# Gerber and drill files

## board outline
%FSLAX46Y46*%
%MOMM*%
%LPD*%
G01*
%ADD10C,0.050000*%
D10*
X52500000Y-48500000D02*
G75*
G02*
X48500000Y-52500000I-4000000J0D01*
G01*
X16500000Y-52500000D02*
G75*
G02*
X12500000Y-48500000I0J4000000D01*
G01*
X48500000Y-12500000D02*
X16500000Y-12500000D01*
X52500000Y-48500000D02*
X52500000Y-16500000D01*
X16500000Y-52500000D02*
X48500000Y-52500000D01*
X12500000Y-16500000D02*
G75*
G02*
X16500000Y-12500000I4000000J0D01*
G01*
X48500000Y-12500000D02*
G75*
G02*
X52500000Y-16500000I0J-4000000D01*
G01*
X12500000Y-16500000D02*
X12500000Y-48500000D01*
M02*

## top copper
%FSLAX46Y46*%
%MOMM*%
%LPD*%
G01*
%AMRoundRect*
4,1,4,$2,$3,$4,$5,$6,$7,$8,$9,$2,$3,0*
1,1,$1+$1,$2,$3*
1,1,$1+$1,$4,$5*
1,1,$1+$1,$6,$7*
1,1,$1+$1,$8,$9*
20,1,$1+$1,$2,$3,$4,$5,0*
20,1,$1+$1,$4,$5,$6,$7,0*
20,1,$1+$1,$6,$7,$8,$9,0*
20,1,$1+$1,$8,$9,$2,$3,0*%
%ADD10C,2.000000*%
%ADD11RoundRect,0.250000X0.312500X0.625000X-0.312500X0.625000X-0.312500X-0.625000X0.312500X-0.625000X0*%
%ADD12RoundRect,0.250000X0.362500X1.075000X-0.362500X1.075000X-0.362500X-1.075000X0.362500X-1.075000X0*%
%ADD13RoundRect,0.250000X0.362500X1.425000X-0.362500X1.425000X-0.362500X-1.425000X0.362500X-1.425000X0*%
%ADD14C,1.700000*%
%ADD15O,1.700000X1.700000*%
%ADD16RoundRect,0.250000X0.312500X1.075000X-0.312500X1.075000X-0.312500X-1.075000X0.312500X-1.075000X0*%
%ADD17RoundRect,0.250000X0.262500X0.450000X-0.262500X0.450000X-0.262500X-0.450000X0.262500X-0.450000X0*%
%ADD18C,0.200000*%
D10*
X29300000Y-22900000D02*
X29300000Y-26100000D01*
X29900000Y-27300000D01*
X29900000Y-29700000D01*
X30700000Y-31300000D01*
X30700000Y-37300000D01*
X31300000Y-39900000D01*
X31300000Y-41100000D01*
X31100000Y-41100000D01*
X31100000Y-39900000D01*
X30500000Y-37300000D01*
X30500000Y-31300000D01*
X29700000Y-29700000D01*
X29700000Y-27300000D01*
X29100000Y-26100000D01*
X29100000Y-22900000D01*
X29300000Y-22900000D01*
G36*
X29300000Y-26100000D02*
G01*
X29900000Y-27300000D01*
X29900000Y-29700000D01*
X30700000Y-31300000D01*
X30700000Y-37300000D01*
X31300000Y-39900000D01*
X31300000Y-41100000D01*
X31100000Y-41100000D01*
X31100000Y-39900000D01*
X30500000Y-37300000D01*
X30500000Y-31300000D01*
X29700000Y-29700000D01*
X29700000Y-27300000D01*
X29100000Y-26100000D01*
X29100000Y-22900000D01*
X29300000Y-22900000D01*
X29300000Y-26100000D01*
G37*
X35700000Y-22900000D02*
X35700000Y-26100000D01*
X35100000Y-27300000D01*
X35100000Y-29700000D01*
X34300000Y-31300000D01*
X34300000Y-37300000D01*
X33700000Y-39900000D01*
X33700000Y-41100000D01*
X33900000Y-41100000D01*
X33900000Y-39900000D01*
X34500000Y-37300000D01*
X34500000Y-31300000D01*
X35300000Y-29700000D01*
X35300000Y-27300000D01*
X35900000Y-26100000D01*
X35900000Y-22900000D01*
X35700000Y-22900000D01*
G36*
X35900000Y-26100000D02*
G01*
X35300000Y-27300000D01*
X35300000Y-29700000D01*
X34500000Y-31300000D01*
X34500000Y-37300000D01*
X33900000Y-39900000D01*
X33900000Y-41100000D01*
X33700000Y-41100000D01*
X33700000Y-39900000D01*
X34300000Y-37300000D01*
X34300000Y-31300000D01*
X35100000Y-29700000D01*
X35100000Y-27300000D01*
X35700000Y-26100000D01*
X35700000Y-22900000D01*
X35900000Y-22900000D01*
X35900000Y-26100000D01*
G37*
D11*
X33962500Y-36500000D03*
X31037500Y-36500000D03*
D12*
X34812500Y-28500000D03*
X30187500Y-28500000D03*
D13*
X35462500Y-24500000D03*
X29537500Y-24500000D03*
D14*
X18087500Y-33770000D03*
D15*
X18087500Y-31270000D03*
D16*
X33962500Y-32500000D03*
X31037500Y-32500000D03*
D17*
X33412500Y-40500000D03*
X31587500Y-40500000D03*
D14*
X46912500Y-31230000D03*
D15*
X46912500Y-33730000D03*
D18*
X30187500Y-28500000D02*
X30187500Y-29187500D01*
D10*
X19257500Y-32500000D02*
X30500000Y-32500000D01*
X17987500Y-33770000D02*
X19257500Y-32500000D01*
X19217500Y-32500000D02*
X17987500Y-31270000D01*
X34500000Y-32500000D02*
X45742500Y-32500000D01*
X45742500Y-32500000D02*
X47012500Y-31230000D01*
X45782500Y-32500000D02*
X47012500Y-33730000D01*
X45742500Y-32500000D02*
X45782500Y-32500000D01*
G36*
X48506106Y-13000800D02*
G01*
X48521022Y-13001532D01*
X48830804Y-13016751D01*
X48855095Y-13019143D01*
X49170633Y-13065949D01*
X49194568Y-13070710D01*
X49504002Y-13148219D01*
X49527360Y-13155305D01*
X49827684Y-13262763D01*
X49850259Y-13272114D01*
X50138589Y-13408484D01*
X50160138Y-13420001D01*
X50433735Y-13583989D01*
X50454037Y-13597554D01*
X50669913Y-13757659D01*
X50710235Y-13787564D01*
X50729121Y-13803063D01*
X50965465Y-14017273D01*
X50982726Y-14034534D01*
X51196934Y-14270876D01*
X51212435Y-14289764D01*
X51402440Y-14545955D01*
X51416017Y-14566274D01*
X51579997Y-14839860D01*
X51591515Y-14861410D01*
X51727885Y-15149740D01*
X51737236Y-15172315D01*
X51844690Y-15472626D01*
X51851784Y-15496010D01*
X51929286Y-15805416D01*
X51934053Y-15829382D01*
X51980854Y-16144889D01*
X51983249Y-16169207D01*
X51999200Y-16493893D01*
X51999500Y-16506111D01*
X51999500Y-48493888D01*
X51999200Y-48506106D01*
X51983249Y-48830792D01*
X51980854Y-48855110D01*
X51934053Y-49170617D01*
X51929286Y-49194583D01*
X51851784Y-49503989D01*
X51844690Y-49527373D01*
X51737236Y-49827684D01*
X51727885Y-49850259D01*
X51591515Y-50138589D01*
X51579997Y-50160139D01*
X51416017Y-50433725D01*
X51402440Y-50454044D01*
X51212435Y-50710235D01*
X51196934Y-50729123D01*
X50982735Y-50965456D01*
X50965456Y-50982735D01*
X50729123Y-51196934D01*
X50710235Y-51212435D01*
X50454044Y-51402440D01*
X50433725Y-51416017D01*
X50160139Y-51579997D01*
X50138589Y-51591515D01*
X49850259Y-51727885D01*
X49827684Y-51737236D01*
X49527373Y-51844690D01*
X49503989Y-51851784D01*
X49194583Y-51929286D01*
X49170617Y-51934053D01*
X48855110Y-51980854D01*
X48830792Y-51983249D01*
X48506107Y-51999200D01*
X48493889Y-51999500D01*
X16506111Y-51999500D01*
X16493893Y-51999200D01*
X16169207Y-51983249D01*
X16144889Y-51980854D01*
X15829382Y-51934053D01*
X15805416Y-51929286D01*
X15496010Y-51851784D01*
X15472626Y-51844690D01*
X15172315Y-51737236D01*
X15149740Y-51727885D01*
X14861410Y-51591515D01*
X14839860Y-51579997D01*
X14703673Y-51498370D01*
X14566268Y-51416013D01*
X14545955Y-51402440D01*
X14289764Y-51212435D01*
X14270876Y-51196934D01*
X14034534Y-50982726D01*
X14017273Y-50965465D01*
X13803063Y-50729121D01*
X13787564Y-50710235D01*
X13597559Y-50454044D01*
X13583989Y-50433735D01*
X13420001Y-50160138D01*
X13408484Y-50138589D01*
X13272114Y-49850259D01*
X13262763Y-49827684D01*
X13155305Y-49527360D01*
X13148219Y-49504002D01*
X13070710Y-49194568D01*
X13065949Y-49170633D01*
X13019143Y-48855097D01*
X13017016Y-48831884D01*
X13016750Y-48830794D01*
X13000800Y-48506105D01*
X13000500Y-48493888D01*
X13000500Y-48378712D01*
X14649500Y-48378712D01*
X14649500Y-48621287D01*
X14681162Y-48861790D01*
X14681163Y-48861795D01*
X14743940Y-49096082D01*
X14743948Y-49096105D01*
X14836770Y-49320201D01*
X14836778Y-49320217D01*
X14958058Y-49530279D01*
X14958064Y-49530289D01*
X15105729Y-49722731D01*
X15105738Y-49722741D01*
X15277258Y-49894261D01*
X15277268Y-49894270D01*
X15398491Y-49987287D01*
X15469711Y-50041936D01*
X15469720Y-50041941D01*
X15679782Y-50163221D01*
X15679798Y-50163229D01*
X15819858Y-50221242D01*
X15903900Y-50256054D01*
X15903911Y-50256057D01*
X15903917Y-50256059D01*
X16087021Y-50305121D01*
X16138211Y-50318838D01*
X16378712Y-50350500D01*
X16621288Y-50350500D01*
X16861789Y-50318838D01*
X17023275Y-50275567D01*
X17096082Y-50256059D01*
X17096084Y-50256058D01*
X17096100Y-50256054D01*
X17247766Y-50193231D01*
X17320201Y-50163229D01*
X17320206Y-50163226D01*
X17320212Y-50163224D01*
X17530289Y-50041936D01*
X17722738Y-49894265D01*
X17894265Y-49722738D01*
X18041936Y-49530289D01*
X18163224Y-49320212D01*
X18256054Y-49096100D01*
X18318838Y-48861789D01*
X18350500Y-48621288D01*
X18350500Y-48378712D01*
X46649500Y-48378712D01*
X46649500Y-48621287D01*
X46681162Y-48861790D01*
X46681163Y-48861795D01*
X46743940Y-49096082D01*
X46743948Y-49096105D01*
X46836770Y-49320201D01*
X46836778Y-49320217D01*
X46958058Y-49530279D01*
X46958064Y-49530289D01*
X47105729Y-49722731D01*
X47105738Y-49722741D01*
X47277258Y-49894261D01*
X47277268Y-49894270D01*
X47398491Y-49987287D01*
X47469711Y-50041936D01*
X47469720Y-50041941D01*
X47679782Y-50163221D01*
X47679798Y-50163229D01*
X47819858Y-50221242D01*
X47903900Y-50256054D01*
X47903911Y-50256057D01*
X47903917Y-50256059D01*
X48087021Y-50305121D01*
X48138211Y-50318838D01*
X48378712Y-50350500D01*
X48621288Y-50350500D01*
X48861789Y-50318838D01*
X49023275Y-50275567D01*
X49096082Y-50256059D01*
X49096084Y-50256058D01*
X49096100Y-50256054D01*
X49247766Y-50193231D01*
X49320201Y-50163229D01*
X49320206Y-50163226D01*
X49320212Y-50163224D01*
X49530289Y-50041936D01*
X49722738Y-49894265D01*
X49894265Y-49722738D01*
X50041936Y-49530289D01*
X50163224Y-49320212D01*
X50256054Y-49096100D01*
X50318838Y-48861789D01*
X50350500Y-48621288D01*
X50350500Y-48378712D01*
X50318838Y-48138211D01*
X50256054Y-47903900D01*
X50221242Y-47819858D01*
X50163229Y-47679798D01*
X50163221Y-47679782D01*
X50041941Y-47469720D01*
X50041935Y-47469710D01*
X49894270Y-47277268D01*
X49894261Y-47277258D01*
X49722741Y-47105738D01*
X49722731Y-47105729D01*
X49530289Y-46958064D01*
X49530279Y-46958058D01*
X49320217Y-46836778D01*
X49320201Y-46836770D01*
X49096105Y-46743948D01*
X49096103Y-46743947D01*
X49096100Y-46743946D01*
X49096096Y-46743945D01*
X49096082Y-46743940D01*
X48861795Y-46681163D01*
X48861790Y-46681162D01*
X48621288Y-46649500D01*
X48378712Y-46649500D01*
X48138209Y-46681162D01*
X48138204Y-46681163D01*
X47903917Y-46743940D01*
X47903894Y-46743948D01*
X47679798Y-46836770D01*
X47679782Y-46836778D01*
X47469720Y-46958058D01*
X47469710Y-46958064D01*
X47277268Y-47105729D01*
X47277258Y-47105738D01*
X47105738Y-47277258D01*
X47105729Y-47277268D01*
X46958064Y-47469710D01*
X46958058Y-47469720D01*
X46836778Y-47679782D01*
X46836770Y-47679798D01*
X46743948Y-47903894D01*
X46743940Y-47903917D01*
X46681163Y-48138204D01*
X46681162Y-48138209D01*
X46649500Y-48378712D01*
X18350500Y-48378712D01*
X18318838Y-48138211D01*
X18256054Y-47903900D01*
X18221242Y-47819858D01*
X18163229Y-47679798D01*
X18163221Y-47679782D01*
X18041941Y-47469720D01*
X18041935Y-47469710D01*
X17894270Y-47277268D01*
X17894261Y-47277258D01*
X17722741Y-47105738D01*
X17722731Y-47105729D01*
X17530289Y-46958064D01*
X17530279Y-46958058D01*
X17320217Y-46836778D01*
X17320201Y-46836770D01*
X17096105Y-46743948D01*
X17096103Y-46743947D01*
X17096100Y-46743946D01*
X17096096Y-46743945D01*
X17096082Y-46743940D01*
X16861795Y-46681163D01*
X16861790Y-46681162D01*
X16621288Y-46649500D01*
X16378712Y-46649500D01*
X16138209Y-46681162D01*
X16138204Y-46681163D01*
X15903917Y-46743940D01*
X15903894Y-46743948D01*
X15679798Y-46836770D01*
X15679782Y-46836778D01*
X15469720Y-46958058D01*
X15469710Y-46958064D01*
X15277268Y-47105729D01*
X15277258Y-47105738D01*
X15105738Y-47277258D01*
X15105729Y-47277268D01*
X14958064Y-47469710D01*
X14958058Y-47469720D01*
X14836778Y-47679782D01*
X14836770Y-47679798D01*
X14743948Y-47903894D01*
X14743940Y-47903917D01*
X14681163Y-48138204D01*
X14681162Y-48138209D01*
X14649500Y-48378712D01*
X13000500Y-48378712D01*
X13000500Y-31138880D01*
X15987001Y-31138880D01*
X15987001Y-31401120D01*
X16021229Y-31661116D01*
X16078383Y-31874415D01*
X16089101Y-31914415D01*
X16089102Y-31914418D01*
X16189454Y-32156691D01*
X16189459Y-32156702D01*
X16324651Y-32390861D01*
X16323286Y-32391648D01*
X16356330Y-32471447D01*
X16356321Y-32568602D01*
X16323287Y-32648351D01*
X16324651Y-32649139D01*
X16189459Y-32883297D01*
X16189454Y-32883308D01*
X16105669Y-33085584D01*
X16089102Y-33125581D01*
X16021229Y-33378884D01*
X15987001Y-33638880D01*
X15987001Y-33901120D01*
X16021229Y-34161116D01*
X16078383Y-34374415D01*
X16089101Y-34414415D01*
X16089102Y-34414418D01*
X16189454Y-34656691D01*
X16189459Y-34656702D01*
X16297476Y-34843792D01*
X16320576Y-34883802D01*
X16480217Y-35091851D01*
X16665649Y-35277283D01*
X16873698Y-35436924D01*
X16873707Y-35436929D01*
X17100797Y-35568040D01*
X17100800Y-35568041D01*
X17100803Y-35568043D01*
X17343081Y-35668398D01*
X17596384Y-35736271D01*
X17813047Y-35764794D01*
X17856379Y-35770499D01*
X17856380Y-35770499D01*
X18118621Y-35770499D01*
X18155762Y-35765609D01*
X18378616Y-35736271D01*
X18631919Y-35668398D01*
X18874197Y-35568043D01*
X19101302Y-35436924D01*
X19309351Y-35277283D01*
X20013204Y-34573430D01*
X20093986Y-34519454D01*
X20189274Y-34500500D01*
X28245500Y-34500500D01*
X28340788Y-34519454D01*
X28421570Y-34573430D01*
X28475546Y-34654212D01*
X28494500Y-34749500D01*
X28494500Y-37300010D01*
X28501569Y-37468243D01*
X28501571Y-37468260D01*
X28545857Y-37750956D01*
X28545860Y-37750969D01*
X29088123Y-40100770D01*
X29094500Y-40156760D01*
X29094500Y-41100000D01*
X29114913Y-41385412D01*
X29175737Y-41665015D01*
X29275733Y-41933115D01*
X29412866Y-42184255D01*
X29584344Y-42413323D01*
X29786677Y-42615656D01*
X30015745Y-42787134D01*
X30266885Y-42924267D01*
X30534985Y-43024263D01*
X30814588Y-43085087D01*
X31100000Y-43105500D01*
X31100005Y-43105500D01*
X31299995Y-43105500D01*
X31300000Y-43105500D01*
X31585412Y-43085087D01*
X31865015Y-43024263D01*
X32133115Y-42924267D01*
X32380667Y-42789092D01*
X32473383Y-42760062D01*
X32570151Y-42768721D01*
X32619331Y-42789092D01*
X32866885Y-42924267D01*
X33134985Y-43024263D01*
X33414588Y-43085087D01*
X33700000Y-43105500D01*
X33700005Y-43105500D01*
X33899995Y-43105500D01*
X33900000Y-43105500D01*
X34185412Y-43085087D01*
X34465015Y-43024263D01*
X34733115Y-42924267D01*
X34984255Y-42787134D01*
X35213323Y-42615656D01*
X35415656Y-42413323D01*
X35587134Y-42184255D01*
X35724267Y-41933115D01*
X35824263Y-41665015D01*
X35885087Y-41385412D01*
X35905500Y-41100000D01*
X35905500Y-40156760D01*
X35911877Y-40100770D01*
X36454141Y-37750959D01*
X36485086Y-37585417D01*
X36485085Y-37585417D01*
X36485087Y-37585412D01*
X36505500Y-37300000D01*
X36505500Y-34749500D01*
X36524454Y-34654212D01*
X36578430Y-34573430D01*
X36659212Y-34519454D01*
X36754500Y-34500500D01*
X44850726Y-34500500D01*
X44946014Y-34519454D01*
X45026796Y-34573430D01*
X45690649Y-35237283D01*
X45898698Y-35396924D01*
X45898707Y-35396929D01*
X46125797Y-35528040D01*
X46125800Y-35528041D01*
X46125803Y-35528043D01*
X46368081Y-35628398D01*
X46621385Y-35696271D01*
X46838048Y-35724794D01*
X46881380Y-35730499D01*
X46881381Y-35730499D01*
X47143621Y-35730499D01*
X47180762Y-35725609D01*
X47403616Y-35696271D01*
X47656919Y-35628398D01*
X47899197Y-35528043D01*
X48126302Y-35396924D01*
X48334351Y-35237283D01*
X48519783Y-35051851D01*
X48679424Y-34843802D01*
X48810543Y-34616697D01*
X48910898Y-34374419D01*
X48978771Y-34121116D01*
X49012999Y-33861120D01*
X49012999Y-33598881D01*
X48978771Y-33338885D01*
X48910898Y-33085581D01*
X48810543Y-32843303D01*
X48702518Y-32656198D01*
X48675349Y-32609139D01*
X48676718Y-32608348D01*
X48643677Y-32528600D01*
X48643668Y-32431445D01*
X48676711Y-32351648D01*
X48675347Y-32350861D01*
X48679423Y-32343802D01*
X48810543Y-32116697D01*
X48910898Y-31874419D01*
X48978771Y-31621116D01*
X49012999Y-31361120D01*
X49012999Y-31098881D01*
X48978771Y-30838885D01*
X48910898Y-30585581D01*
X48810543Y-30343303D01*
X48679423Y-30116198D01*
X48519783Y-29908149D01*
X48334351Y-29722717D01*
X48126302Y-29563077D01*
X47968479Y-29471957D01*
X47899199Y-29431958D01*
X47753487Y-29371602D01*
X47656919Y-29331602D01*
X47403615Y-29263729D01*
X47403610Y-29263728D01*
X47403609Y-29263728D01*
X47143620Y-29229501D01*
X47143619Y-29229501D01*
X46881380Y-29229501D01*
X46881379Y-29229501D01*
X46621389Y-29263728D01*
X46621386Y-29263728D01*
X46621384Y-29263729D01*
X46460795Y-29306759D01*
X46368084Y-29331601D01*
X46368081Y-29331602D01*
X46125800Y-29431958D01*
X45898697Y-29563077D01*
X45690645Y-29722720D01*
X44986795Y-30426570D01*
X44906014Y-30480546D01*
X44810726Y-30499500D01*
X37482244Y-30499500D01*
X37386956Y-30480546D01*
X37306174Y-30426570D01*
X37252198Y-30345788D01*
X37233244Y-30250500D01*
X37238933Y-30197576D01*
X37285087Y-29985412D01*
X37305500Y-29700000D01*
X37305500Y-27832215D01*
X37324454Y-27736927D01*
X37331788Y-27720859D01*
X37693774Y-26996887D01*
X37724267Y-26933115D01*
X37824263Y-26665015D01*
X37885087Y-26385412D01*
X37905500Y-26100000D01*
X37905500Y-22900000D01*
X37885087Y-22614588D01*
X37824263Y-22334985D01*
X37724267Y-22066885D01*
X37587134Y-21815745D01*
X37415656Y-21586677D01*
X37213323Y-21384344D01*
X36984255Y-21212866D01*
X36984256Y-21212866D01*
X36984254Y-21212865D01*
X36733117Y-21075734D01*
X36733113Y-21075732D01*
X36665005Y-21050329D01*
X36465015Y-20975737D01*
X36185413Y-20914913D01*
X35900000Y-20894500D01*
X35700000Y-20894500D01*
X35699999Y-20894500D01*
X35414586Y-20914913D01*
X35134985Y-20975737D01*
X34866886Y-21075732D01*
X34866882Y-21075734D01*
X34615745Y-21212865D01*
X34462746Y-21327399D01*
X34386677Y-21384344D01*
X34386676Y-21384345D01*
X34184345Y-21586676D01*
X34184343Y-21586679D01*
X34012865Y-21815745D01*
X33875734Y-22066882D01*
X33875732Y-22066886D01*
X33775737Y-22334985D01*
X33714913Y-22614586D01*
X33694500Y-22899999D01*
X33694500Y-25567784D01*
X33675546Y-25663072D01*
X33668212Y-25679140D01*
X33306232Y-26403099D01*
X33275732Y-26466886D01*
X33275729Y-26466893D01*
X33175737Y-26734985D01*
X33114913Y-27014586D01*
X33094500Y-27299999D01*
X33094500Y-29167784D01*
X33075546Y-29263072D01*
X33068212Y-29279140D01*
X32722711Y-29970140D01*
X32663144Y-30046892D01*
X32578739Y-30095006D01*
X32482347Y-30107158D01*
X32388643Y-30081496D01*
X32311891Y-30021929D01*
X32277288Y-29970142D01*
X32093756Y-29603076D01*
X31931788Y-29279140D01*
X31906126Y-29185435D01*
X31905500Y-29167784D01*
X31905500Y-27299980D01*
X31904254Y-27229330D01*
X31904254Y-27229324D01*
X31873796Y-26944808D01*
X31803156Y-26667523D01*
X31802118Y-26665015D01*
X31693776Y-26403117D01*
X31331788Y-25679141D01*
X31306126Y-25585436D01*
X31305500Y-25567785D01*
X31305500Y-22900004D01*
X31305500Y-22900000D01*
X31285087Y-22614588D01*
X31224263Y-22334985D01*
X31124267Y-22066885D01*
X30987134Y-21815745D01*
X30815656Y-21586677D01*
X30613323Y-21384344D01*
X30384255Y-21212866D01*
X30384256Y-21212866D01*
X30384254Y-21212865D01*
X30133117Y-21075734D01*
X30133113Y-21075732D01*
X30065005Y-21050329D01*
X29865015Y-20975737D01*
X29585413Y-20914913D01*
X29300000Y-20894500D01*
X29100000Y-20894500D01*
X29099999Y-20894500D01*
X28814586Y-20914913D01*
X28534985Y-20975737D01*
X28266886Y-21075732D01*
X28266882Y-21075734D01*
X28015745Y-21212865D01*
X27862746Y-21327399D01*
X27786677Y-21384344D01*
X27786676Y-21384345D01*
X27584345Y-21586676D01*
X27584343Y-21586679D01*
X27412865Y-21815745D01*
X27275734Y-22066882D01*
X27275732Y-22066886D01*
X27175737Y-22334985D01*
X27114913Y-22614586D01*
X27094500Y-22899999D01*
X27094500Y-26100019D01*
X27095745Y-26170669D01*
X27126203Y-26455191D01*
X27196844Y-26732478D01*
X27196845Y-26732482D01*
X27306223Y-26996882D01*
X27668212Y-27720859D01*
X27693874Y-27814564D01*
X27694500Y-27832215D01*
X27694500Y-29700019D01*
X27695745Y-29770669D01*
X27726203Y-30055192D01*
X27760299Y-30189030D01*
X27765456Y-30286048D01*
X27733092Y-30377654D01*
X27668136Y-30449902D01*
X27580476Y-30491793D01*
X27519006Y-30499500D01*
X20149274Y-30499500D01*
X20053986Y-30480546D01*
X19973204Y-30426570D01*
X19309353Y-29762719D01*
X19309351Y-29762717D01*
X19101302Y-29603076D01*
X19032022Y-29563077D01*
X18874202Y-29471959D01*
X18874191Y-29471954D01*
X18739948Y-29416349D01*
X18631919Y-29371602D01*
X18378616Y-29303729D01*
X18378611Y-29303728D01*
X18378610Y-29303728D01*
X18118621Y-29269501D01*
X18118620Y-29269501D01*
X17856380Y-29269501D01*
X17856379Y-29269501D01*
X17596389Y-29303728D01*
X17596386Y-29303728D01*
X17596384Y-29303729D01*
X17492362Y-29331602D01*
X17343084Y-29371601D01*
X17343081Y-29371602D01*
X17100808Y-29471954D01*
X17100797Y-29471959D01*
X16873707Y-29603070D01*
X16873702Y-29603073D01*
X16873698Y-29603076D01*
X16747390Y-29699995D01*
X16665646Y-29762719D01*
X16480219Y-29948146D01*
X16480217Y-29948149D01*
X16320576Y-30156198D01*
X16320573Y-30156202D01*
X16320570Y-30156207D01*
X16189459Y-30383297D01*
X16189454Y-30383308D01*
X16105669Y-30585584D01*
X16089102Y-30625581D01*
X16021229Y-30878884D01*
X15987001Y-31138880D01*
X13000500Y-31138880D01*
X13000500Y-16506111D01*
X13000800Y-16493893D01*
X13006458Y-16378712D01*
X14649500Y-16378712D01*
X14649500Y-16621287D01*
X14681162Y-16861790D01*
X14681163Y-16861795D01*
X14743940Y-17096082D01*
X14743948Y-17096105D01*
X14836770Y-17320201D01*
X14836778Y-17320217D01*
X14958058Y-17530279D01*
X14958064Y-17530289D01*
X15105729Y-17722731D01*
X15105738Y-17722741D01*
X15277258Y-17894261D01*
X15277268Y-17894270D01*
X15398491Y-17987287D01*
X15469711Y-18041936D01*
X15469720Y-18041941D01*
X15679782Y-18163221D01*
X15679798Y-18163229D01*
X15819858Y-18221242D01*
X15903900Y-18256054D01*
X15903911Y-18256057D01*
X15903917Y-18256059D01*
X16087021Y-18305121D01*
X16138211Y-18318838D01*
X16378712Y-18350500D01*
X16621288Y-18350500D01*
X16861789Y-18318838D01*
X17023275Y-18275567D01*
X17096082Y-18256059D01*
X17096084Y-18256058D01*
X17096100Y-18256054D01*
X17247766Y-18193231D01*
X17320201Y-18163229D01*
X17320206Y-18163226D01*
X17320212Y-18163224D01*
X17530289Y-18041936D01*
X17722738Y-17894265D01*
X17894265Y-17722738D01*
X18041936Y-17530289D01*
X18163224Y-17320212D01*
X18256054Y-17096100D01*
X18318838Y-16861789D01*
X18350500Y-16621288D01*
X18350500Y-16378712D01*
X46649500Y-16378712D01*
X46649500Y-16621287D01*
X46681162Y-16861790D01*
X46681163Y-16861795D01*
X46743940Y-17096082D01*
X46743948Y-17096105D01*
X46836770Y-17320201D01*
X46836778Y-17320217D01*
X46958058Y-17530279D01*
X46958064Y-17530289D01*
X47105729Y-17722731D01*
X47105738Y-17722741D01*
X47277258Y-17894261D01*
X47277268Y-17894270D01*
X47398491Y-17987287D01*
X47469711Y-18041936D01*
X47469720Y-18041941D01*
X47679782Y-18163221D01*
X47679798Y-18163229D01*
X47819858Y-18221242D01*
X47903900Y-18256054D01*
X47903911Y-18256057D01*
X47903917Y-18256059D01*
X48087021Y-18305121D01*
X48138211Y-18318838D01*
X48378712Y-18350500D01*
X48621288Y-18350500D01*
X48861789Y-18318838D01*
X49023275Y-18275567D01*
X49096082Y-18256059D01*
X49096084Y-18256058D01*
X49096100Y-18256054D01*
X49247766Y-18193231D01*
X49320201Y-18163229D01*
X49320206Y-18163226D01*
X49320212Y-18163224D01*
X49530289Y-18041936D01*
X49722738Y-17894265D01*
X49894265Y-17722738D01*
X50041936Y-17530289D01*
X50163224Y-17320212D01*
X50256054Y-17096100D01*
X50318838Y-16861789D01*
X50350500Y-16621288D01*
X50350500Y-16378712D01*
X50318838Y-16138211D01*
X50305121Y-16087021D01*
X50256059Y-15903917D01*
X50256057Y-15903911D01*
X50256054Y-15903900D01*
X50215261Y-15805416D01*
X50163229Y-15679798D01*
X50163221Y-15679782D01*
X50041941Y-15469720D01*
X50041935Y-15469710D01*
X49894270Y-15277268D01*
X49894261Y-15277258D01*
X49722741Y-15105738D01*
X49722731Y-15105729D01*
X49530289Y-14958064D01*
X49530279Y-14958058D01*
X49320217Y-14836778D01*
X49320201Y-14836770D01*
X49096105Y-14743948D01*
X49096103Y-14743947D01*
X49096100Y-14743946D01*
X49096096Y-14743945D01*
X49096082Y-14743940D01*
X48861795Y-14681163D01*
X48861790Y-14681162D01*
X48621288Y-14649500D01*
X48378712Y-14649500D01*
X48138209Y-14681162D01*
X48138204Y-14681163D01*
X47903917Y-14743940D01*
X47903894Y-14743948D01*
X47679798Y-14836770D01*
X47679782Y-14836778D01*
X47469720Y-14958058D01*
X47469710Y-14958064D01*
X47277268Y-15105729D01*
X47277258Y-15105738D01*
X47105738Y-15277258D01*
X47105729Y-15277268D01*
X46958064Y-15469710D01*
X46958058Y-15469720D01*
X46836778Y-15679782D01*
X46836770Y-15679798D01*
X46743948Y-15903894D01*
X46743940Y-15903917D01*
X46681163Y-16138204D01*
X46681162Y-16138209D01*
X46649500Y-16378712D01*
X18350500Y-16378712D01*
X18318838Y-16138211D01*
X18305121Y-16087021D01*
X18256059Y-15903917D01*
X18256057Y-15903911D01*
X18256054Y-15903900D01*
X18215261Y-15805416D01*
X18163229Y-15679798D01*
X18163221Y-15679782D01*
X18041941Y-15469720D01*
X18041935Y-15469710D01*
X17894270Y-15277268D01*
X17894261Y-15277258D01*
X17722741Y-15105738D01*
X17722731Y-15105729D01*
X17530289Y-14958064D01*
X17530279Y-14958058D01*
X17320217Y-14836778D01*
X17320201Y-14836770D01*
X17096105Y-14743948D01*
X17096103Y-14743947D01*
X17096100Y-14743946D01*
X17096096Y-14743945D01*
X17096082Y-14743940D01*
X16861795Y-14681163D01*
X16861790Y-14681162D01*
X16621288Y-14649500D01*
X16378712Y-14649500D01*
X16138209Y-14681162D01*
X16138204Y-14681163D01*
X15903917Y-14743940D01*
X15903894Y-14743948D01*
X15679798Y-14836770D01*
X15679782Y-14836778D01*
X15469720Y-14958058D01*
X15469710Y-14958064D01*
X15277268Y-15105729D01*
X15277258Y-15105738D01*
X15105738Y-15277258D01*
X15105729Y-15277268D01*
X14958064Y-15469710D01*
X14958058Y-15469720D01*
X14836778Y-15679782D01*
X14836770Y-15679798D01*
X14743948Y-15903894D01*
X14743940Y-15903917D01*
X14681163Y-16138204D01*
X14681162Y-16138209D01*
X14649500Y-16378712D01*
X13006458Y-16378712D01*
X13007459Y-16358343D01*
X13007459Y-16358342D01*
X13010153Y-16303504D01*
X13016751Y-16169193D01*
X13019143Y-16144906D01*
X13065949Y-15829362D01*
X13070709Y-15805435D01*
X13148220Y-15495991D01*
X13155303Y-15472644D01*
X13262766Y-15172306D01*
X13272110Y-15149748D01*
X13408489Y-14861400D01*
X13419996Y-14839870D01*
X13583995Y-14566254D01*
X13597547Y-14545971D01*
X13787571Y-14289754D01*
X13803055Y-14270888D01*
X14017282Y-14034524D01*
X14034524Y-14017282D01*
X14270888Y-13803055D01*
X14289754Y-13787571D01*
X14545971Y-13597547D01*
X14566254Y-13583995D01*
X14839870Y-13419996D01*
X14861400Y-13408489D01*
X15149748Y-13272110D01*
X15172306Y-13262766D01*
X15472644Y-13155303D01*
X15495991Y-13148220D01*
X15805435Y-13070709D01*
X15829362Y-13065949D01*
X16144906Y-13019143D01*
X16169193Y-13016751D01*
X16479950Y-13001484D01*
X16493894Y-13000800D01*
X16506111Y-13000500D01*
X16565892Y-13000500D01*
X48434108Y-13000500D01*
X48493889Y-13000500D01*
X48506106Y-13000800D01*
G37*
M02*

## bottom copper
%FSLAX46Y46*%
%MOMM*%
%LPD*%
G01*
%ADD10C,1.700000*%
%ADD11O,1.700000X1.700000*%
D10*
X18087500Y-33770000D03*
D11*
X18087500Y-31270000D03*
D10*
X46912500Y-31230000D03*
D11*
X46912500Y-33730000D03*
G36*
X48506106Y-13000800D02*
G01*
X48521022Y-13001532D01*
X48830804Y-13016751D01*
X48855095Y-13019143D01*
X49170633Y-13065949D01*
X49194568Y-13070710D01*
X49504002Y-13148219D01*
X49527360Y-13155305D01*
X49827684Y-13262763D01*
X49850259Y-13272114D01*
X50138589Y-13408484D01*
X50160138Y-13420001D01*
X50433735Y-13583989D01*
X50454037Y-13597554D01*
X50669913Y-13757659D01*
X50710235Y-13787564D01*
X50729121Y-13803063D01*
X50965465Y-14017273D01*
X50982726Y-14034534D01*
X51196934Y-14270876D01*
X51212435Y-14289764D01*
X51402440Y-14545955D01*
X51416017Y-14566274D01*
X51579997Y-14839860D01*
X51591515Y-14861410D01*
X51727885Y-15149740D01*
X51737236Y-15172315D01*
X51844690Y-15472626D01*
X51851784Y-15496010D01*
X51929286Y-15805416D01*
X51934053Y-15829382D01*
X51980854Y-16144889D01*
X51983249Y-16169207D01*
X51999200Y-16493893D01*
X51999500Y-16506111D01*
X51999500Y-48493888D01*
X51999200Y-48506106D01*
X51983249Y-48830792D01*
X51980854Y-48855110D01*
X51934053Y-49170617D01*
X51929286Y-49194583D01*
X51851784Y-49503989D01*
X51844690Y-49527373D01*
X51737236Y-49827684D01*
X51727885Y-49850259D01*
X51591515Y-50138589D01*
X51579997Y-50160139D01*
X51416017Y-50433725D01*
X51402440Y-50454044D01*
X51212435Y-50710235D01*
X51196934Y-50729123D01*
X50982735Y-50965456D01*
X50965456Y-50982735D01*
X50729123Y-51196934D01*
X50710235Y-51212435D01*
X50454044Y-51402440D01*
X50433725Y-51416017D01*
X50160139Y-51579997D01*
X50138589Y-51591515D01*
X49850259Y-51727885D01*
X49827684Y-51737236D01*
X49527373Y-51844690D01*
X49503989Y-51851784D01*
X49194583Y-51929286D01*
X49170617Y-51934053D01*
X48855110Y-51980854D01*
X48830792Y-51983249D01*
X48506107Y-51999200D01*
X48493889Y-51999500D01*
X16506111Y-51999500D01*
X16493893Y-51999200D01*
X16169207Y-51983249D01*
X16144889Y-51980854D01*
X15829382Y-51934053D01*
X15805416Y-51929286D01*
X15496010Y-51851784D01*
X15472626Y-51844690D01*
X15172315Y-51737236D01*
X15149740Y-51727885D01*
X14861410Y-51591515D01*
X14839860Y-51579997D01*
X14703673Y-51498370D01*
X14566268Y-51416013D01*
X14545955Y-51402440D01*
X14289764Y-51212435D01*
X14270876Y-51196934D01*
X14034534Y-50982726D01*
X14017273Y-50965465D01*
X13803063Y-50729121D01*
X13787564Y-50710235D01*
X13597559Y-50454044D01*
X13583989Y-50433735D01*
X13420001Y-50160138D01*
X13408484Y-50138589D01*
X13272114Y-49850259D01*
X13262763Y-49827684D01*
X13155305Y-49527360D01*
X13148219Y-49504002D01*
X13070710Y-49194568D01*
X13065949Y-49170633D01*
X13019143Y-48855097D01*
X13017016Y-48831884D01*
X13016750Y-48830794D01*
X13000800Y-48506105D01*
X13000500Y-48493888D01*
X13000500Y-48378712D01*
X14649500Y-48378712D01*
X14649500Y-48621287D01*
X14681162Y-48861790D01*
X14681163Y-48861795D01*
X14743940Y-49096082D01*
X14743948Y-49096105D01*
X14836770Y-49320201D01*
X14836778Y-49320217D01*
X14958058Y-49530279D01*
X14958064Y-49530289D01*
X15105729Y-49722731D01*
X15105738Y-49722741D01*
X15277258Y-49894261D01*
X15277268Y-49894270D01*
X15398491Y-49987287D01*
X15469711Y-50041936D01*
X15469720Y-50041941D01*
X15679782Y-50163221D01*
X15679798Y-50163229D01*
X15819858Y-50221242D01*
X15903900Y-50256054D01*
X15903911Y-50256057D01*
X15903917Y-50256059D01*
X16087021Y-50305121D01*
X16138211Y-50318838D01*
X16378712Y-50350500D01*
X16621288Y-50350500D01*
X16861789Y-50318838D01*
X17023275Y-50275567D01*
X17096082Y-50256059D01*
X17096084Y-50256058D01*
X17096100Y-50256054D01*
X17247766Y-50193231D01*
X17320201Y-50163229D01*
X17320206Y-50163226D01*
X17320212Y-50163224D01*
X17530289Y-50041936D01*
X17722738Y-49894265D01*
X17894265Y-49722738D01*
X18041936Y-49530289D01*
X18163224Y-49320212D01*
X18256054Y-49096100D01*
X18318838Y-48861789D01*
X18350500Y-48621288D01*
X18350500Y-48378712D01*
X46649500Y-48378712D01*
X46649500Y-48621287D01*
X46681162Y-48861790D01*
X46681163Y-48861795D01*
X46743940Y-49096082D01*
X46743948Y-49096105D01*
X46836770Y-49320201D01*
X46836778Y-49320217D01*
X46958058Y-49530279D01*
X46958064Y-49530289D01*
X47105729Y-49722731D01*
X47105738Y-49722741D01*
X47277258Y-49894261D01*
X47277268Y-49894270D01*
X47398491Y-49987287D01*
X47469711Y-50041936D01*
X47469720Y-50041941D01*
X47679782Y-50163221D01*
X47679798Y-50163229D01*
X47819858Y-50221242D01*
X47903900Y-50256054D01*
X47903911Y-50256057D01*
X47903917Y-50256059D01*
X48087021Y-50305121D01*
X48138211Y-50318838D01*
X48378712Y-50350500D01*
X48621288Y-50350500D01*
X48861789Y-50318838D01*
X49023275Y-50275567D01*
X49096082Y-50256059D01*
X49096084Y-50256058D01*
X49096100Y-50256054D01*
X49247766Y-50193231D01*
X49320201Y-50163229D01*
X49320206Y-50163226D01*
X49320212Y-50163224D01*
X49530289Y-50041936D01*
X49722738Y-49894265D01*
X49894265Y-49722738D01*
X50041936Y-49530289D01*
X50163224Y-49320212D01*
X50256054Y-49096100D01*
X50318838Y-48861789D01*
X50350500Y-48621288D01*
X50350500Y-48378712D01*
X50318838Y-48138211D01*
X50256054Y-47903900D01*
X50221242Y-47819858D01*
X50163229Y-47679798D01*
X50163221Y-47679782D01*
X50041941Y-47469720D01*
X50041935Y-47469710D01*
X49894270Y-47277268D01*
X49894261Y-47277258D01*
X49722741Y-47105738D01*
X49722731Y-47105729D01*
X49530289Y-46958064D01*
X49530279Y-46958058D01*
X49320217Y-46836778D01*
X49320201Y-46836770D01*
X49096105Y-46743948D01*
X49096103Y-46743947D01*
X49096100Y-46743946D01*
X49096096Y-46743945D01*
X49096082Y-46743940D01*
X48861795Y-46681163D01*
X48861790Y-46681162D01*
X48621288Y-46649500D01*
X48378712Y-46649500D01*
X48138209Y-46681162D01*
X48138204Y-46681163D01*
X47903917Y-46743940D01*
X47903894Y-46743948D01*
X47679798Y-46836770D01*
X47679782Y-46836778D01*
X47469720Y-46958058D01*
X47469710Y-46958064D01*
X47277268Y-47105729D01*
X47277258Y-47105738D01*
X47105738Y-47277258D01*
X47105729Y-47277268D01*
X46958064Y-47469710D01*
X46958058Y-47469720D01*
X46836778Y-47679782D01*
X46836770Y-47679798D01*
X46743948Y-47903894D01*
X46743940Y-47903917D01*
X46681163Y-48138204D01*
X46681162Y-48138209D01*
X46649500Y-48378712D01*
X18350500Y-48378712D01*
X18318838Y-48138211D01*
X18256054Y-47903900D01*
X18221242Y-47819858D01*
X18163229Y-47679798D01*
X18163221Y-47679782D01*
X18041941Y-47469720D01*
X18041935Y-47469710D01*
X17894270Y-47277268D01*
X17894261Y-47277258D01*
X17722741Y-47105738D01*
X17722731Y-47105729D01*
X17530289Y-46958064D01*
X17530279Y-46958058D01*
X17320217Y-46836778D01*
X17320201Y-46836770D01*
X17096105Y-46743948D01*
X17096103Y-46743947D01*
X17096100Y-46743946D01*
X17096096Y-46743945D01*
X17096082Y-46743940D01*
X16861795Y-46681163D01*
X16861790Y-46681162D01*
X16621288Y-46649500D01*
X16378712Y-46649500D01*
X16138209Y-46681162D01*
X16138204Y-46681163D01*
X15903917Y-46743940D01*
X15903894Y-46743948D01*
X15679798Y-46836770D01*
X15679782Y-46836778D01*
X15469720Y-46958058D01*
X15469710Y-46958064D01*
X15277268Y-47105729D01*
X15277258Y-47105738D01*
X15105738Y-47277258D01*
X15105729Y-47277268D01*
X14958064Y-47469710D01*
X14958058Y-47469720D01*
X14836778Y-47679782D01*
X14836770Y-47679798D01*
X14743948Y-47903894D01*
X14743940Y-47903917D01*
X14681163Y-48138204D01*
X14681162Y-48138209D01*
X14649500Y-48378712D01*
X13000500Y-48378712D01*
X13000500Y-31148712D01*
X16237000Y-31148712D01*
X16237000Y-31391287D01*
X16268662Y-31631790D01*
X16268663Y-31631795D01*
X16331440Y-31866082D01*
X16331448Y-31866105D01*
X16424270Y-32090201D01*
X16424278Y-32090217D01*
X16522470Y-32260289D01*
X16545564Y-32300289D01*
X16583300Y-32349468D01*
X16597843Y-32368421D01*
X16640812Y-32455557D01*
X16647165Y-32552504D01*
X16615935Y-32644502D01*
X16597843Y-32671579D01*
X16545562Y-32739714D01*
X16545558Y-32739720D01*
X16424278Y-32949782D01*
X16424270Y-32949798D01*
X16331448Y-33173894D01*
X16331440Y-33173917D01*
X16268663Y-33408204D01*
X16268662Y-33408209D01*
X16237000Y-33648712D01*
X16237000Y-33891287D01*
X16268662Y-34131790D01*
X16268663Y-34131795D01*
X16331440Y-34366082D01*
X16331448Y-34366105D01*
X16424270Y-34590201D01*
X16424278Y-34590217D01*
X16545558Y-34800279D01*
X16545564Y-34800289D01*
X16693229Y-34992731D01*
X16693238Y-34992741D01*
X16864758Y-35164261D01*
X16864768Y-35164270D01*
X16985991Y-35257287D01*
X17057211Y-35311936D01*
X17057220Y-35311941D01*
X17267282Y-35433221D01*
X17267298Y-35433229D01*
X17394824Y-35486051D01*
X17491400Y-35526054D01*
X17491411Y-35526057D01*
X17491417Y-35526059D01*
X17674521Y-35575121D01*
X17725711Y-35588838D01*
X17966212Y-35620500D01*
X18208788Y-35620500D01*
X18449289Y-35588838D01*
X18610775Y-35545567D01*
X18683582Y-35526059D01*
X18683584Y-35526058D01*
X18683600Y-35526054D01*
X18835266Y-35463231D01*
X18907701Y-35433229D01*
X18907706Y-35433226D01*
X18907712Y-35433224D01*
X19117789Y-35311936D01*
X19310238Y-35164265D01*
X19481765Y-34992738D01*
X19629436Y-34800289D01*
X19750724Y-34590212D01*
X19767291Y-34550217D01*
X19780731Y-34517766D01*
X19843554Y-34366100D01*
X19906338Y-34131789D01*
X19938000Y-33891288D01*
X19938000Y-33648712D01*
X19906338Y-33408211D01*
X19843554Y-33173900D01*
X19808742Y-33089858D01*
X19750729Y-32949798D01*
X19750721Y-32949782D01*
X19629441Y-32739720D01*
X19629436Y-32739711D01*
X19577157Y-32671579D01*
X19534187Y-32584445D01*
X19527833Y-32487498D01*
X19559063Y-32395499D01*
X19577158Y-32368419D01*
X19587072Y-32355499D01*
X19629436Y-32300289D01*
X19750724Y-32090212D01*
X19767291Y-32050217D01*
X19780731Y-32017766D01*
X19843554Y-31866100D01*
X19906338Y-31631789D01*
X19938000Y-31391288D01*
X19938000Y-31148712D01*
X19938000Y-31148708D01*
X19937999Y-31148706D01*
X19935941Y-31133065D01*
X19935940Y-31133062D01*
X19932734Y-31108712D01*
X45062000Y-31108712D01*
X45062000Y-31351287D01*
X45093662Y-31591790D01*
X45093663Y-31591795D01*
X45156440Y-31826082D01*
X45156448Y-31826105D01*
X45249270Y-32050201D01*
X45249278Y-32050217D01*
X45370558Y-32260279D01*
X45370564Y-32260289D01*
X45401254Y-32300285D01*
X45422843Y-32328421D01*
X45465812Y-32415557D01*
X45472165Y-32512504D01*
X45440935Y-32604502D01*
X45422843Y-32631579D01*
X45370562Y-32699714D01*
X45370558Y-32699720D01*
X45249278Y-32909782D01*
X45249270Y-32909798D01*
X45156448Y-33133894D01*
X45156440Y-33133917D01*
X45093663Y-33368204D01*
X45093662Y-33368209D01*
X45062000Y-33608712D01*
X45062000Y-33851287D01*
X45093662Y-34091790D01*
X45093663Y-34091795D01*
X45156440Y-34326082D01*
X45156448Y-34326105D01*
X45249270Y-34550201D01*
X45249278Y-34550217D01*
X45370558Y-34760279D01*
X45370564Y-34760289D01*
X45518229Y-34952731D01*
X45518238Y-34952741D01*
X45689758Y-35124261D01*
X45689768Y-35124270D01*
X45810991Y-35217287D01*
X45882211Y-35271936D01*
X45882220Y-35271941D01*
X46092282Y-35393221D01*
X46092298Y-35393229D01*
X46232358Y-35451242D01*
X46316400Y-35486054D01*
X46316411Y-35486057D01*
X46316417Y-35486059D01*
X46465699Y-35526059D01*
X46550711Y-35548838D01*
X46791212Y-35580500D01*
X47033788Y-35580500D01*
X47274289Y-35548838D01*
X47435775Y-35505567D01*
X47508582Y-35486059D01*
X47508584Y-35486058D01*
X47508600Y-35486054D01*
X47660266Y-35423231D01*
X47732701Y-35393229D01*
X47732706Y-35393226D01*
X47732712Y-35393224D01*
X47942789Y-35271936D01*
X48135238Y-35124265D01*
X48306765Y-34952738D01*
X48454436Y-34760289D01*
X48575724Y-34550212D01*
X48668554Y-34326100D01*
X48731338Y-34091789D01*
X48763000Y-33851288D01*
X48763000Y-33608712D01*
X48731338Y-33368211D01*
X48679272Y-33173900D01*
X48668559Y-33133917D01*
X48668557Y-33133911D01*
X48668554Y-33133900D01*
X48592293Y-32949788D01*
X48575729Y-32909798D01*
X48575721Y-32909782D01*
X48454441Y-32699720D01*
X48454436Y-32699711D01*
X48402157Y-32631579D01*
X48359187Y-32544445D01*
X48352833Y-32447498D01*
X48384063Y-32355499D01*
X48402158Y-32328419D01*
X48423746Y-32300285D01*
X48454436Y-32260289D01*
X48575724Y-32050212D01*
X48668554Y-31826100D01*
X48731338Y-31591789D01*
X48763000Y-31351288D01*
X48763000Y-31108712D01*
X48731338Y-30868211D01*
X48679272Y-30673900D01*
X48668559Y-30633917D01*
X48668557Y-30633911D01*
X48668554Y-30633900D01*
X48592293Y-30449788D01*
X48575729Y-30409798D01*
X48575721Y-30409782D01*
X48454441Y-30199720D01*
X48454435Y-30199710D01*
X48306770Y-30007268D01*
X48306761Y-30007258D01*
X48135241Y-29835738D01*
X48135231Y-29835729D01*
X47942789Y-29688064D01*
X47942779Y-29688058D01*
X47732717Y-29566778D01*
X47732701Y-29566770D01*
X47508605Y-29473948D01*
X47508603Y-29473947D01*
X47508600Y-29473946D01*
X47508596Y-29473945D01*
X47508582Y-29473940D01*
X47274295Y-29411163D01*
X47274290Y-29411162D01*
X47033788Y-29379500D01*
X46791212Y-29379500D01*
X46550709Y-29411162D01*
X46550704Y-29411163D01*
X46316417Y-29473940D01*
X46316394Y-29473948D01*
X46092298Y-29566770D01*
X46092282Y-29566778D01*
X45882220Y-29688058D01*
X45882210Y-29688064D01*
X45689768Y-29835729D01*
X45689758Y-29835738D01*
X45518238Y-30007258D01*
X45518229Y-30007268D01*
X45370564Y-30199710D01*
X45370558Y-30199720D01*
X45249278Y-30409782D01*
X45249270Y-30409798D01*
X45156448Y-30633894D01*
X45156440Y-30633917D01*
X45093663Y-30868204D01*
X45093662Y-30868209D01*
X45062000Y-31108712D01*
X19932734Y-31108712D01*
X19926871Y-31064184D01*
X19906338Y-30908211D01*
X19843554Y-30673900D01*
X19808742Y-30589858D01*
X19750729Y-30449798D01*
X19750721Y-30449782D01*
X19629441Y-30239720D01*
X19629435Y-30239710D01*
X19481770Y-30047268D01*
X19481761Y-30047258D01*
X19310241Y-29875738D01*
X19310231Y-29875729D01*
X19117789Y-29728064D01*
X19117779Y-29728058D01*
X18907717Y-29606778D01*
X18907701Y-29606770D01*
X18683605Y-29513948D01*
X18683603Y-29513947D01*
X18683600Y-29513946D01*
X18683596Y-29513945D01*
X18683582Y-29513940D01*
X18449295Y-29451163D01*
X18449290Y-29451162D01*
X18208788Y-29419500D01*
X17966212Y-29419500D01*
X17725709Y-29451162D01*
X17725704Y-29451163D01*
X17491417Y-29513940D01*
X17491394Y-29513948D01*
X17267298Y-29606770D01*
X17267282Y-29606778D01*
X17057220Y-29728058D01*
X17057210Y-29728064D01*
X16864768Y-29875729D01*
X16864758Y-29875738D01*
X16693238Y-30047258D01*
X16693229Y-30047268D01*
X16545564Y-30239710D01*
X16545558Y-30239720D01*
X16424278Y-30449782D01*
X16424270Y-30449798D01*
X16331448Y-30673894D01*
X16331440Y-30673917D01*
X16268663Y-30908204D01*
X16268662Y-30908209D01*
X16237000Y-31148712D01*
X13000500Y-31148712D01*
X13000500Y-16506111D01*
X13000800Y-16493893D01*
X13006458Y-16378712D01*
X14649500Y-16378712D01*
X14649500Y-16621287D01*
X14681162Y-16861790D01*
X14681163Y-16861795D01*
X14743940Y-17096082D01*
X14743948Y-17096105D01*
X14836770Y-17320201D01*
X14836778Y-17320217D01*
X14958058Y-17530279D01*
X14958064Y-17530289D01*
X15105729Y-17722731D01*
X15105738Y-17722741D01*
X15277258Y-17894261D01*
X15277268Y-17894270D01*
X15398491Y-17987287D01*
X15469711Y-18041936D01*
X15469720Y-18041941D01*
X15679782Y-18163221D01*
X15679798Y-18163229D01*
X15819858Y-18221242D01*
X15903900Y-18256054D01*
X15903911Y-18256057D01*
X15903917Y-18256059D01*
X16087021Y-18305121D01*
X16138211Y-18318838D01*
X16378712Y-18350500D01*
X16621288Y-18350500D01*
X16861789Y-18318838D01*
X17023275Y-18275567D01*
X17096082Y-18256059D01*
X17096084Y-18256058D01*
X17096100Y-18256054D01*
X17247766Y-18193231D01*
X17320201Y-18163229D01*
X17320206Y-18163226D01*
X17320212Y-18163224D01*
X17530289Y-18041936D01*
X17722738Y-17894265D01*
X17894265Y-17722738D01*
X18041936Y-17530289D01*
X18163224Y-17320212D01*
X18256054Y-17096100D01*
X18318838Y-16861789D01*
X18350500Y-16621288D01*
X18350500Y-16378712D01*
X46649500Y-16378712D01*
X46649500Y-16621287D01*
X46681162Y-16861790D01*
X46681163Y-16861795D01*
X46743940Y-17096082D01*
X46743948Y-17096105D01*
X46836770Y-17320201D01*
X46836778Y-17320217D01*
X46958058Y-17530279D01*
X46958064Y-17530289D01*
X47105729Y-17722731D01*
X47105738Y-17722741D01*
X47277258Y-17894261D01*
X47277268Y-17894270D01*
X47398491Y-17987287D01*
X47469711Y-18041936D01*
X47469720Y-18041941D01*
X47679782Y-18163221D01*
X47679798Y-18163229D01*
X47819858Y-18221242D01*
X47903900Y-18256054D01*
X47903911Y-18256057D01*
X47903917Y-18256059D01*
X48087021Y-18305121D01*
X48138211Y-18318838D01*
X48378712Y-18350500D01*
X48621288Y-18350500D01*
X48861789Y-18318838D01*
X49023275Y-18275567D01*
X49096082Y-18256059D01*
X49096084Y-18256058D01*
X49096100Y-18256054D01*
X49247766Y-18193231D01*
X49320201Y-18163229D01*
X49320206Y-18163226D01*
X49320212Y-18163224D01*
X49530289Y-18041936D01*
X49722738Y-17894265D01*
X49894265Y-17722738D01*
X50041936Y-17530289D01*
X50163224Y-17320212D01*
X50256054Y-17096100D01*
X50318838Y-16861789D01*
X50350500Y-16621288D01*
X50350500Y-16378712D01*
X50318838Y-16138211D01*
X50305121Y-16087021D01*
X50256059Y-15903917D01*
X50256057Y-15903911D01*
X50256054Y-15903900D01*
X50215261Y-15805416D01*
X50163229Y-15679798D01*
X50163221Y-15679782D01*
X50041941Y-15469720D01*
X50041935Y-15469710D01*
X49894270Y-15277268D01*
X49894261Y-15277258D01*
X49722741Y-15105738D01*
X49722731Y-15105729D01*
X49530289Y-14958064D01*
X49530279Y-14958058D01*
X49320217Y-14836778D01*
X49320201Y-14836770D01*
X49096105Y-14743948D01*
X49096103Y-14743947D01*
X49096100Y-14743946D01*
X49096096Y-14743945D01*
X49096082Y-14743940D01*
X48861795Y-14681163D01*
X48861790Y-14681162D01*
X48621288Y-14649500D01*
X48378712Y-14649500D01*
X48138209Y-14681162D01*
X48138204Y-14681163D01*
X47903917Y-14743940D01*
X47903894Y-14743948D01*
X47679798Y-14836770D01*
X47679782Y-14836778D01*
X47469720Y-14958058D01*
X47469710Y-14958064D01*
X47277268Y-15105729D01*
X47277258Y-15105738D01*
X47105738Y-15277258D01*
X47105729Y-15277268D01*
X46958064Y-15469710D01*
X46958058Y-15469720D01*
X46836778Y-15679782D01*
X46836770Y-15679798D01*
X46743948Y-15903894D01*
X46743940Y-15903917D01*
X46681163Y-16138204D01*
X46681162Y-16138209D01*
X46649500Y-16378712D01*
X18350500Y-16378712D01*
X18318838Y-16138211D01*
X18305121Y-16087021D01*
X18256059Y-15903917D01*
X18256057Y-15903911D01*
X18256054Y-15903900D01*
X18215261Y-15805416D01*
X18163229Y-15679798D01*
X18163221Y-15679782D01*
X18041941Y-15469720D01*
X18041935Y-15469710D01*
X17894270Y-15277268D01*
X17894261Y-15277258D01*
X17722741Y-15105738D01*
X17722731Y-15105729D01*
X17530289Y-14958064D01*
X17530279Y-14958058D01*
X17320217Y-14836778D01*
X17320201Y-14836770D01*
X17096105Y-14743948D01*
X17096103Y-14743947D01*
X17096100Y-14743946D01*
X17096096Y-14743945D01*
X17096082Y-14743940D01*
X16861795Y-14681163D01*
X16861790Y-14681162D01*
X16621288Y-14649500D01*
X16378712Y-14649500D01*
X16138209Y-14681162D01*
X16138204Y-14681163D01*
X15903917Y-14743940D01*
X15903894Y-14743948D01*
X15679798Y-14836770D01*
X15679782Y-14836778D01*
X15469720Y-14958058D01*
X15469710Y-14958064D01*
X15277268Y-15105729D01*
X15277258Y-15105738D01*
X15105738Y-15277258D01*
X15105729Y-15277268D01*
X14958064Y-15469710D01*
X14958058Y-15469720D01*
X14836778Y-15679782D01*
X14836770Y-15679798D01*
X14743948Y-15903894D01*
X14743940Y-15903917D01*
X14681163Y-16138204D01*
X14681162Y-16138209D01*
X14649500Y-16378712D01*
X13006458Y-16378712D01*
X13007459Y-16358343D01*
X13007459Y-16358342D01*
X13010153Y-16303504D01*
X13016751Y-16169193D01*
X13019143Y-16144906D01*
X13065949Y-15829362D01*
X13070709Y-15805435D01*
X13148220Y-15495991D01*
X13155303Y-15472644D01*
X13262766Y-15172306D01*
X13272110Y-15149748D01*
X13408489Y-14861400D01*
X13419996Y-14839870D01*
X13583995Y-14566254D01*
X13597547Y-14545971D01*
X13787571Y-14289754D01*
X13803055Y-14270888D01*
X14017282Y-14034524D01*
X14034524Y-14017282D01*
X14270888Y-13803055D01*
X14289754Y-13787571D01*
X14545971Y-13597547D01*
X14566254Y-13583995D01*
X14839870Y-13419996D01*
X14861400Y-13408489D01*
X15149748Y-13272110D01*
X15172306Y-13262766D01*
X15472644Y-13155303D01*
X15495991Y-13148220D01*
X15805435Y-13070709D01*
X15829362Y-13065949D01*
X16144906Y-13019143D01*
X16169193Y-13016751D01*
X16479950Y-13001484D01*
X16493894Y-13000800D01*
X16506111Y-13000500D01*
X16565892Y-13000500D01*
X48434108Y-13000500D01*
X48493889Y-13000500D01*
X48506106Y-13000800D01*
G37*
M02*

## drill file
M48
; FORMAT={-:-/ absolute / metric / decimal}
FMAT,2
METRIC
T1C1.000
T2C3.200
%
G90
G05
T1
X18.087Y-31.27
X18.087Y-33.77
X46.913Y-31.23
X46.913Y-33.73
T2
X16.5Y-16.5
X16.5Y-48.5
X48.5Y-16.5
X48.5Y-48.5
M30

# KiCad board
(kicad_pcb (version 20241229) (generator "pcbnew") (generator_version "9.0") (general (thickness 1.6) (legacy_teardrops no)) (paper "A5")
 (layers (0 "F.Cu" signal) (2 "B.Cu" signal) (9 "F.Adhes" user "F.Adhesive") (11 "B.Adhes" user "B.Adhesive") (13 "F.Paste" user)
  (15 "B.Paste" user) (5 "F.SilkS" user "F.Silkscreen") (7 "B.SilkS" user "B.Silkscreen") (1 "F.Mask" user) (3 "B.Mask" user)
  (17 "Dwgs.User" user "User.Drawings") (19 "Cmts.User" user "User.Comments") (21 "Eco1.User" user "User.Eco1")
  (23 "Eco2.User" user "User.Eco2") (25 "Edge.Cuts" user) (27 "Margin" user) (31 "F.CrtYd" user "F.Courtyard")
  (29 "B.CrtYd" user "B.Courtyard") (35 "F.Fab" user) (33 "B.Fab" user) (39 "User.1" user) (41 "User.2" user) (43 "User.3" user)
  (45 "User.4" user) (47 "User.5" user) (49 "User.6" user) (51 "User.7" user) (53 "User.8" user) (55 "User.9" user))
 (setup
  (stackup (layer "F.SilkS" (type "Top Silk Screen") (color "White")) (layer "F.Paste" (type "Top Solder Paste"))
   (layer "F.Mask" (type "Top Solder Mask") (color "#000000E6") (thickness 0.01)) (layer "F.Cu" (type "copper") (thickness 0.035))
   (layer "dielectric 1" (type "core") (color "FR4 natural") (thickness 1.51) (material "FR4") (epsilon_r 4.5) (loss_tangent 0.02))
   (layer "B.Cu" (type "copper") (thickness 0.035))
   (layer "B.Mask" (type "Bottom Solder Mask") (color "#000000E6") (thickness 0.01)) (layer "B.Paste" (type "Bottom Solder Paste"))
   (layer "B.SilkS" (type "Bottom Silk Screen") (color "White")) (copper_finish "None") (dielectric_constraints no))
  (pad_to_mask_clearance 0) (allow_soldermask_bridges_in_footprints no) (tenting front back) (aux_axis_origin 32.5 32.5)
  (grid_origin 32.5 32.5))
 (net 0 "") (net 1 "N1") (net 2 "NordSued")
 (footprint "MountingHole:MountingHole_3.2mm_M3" (layer "F.Cu") (at 48.5 48.5 -90)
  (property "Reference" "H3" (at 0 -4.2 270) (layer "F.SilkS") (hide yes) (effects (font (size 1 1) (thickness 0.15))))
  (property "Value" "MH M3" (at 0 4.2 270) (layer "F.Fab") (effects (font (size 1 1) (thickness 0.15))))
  (pad "" np_thru_hole circle (at 0 0 270) (size 3.2 3.2) (drill 3.2) (layers "*.Cu" "*.Mask")))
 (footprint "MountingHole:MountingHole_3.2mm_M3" (layer "F.Cu") (at 48.5 16.5 -90)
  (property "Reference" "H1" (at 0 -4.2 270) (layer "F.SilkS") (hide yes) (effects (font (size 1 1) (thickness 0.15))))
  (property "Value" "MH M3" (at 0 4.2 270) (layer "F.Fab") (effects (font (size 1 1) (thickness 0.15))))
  (pad "" np_thru_hole circle (at 0 0 270) (size 3.2 3.2) (drill 3.2) (layers "*.Cu" "*.Mask")))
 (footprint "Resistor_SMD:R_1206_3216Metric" (layer "F.Cu") (at 32.5 36.5 180)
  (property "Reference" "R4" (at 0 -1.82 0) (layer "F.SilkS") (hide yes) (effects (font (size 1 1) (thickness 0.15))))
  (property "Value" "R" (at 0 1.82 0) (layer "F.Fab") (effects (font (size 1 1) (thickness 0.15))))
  (pad "1" smd roundrect (at -1.4625 0 180) (size 1.125 1.75) (layers "F.Cu" "F.Mask" "F.Paste") (roundrect_rratio 0.222222) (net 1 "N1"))
  (pad "2" smd roundrect (at 1.4625 0 180) (size 1.125 1.75) (layers "F.Cu" "F.Mask" "F.Paste") (roundrect_rratio 0.222222)
   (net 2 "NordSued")))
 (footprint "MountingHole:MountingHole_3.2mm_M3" (layer "F.Cu") (at 16.5 48.5 -90)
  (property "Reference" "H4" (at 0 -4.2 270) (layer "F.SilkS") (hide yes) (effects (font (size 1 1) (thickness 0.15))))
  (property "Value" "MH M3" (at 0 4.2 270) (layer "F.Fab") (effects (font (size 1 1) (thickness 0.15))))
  (pad "" np_thru_hole circle (at 0 0 270) (size 3.2 3.2) (drill 3.2) (layers "*.Cu" "*.Mask")))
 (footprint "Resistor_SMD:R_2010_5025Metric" (layer "F.Cu") (at 32.5 28.5 180)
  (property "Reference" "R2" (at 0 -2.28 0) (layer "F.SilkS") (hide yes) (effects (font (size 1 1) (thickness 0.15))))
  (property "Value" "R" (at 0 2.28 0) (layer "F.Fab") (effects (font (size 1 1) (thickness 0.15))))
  (pad "1" smd roundrect (at -2.3125 0 180) (size 1.225 2.65) (layers "F.Cu" "F.Mask" "F.Paste") (roundrect_rratio 0.204082) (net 1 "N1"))
  (pad "2" smd roundrect (at 2.3125 0 180) (size 1.225 2.65) (layers "F.Cu" "F.Mask" "F.Paste") (roundrect_rratio 0.204082)
   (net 2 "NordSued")))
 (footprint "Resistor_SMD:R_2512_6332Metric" (layer "F.Cu") (at 32.5 24.5 180)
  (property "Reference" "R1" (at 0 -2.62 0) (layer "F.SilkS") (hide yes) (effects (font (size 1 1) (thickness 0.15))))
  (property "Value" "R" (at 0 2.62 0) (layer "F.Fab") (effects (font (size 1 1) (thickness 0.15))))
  (pad "1" smd roundrect (at -2.9625 0 180) (size 1.225 3.35) (layers "F.Cu" "F.Mask" "F.Paste") (roundrect_rratio 0.204082) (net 1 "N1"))
  (pad "2" smd roundrect (at 2.9625 0 180) (size 1.225 3.35) (layers "F.Cu" "F.Mask" "F.Paste") (roundrect_rratio 0.204082)
   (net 2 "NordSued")))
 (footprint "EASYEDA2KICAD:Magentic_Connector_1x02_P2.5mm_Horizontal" (layer "F.Cu") (at 17.9875 32.5 180)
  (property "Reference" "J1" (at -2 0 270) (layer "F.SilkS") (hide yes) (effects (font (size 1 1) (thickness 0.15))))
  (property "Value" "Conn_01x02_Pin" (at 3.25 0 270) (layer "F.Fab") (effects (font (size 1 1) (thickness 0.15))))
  (pad "1" thru_hole circle (at -0.1 -1.27 180) (size 1.7 1.7) (drill 1) (layers "*.Cu" "*.Mask") (remove_unused_layers no)
   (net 2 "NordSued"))
  (pad "2" thru_hole oval (at -0.1 1.23 180) (size 1.7 1.7) (drill 1) (layers "*.Cu" "*.Mask") (remove_unused_layers no) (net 2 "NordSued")))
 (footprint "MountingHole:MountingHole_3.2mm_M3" (layer "F.Cu") (at 16.5 16.5 -90)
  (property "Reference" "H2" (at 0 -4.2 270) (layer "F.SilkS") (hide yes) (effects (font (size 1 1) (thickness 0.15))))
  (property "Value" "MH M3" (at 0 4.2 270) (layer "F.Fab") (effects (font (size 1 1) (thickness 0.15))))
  (pad "" np_thru_hole circle (at 0 0 270) (size 3.2 3.2) (drill 3.2) (layers "*.Cu" "*.Mask")))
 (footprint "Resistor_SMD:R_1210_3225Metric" (layer "F.Cu") (at 32.5 32.5 180)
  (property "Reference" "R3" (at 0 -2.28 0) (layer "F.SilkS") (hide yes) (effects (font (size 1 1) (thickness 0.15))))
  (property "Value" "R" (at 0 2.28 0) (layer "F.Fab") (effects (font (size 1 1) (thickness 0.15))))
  (pad "1" smd roundrect (at -1.4625 0 180) (size 1.125 2.65) (layers "F.Cu" "F.Mask" "F.Paste") (roundrect_rratio 0.222222) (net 1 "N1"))
  (pad "2" smd roundrect (at 1.4625 0 180) (size 1.125 2.65) (layers "F.Cu" "F.Mask" "F.Paste") (roundrect_rratio 0.222222)
   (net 2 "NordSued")))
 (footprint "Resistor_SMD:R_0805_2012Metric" (layer "F.Cu") (at 32.5 40.5 180)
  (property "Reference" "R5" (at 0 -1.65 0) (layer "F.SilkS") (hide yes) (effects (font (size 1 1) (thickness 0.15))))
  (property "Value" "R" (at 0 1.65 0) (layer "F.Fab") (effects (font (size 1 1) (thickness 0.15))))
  (pad "1" smd roundrect (at -0.9125 0 180) (size 1.025 1.4) (layers "F.Cu" "F.Mask" "F.Paste") (roundrect_rratio 0.243902) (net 1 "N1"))
  (pad "2" smd roundrect (at 0.9125 0 180) (size 1.025 1.4) (layers "F.Cu" "F.Mask" "F.Paste") (roundrect_rratio 0.243902)
   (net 2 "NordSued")))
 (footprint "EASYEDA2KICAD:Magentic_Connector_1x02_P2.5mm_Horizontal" (layer "F.Cu") (at 47.0125 32.5)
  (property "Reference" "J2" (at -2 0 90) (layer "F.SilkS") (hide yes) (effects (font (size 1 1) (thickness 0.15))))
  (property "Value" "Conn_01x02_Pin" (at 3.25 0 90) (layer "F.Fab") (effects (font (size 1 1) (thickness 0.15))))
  (pad "1" thru_hole circle (at -0.1 -1.27) (size 1.7 1.7) (drill 1) (layers "*.Cu" "*.Mask") (remove_unused_layers no) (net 1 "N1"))
  (pad "2" thru_hole oval (at -0.1 1.23) (size 1.7 1.7) (drill 1) (layers "*.Cu" "*.Mask") (remove_unused_layers no) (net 1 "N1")))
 (gr_poly
  (pts (xy 29.3 22.9) (xy 29.3 26.1) (xy 29.9 27.3) (xy 29.9 29.7) (xy 30.7 31.3) (xy 30.7 37.3) (xy 31.3 39.9) (xy 31.3 41.1)
   (xy 31.1 41.1) (xy 31.1 39.9) (xy 30.5 37.3) (xy 30.5 31.3) (xy 29.7 29.7) (xy 29.7 27.3) (xy 29.1 26.1) (xy 29.1 22.9))
  (stroke (width 2) (type solid)) (fill yes) (layer "F.Cu") (net 2))
 (gr_poly
  (pts (xy 35.7 22.9) (xy 35.7 26.1) (xy 35.1 27.3) (xy 35.1 29.7) (xy 34.3 31.3) (xy 34.3 37.3) (xy 33.7 39.9) (xy 33.7 41.1)
   (xy 33.9 41.1) (xy 33.9 39.9) (xy 34.5 37.3) (xy 34.5 31.3) (xy 35.3 29.7) (xy 35.3 27.3) (xy 35.9 26.1) (xy 35.9 22.9))
  (stroke (width 2) (type solid)) (fill yes) (layer "F.Cu") (net 1))
 (gr_arc (start 52.5 48.5) (mid 51.328427 51.328427) (end 48.5 52.5) (stroke (width 0.05) (type default)) (layer "Edge.Cuts"))
 (gr_arc (start 16.5 52.5) (mid 13.671573 51.328427) (end 12.5 48.5) (stroke (width 0.05) (type default)) (layer "Edge.Cuts"))
 (gr_line (start 48.5 12.5) (end 16.5 12.5) (stroke (width 0.05) (type default)) (layer "Edge.Cuts"))
 (gr_line (start 52.5 48.5) (end 52.5 16.5) (stroke (width 0.05) (type default)) (layer "Edge.Cuts"))
 (gr_line (start 16.5 52.5) (end 48.5 52.5) (stroke (width 0.05) (type default)) (layer "Edge.Cuts"))
 (gr_arc (start 12.5 16.5) (mid 13.671573 13.671573) (end 16.5 12.5) (stroke (width 0.05) (type default)) (layer "Edge.Cuts"))
 (gr_arc (start 48.5 12.5) (mid 51.328427 13.671573) (end 52.5 16.5) (stroke (width 0.05) (type default)) (layer "Edge.Cuts"))
 (gr_line (start 12.5 16.5) (end 12.5 48.5) (stroke (width 0.05) (type default)) (layer "Edge.Cuts"))
 (segment (start 30.1875 28.5) (end 30.1875 29.1875) (width 0.2) (layer "F.Cu") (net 2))
 (segment (start 19.2575 32.5) (end 30.5 32.5) (width 2) (layer "F.Cu") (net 2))
 (segment (start 17.9875 33.77) (end 19.2575 32.5) (width 2) (layer "F.Cu") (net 2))
 (segment (start 19.2175 32.5) (end 17.9875 31.27) (width 2) (layer "F.Cu") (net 2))
 (segment (start 34.5 32.5) (end 45.7425 32.5) (width 2) (layer "F.Cu") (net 1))
 (segment (start 45.7425 32.5) (end 47.0125 31.23) (width 2) (layer "F.Cu") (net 1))
 (segment (start 45.7825 32.5) (end 47.0125 33.73) (width 2) (layer "F.Cu") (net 1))
 (segment (start 45.7425 32.5) (end 45.7825 32.5) (width 2) (layer "F.Cu") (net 1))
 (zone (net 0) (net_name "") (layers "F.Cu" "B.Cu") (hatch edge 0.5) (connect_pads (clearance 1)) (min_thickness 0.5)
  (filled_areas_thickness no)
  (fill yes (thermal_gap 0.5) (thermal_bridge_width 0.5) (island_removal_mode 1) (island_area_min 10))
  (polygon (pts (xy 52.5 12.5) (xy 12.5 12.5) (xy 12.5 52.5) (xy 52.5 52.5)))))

